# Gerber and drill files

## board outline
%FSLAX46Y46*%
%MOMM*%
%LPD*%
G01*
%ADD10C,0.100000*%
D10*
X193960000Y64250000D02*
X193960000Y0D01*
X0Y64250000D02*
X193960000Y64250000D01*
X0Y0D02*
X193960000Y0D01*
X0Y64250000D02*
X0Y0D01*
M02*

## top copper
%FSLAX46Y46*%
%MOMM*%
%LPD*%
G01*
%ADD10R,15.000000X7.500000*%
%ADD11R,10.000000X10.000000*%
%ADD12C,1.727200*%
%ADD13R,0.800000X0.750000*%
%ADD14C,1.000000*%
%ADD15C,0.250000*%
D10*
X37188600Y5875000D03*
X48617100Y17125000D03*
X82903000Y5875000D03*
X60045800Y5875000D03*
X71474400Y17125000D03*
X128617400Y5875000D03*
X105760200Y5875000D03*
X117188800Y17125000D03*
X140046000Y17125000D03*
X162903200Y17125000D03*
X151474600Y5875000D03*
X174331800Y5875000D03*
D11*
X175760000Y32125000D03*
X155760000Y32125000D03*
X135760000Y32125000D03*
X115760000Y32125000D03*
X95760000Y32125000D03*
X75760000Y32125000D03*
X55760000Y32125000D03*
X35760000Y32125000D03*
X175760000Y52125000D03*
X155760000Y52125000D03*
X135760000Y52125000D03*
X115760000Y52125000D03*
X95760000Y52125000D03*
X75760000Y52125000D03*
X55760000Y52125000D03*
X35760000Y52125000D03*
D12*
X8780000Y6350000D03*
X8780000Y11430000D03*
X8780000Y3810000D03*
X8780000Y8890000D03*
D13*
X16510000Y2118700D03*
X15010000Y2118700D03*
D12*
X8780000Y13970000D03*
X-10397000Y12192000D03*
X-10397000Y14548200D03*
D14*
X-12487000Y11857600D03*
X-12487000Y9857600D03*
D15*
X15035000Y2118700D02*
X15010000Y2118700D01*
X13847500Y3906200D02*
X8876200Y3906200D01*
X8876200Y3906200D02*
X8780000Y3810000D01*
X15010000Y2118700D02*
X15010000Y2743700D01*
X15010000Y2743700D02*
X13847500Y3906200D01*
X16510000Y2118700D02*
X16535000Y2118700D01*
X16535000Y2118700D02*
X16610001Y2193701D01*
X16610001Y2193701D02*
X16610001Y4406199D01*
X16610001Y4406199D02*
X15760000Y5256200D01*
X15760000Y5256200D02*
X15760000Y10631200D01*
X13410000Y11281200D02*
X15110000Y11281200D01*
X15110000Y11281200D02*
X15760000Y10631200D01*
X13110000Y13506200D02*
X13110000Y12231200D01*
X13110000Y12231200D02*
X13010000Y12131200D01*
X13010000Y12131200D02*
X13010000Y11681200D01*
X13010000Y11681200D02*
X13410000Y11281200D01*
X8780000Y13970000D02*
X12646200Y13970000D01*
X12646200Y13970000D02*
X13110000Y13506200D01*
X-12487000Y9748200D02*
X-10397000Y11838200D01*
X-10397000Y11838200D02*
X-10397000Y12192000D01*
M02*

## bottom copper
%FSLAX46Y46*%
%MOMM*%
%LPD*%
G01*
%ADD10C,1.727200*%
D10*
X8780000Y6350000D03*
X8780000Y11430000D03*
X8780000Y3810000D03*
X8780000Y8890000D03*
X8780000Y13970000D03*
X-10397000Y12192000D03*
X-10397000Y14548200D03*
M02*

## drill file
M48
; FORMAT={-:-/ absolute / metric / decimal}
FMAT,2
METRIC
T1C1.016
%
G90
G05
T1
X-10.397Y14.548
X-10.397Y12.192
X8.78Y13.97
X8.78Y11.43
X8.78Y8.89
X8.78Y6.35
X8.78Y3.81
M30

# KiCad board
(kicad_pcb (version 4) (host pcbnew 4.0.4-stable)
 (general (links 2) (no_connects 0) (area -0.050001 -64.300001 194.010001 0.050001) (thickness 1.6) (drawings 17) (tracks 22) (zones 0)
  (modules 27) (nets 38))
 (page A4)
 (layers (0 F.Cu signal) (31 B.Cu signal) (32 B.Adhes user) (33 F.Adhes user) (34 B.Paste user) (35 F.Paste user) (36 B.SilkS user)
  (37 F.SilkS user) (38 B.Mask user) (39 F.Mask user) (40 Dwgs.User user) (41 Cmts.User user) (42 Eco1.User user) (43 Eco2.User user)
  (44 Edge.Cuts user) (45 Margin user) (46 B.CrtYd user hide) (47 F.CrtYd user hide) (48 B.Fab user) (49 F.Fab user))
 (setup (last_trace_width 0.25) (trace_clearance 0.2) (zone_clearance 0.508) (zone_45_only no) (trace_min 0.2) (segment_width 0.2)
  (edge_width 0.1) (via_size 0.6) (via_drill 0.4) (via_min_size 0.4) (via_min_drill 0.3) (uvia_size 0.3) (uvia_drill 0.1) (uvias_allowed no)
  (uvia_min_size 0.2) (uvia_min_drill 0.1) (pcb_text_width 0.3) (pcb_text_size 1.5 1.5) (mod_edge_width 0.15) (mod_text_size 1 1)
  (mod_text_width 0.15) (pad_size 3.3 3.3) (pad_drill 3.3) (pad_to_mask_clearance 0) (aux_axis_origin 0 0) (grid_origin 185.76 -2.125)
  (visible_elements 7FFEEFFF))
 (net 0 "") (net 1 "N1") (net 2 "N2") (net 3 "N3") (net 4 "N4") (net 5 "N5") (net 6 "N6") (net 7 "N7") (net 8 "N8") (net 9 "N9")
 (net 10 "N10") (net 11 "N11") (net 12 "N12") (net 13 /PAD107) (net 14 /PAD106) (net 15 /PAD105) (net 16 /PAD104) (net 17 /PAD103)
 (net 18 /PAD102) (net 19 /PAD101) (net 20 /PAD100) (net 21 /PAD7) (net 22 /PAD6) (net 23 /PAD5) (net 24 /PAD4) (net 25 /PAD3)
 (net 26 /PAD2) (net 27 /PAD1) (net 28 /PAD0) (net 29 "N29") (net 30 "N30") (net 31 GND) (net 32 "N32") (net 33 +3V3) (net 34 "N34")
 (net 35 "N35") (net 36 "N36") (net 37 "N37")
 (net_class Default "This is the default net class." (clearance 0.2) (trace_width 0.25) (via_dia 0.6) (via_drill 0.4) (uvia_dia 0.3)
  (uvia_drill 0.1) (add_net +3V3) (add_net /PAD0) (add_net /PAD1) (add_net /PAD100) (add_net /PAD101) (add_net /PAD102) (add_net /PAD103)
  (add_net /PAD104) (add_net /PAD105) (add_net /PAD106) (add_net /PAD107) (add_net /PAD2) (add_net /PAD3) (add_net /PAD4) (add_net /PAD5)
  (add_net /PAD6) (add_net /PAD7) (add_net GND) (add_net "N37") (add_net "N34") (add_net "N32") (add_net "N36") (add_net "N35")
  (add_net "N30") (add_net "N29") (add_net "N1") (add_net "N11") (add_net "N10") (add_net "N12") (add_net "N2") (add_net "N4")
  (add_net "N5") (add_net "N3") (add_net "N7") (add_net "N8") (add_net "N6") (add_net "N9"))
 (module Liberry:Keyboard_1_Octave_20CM (layer F.Cu) (at 25.76 -2.125)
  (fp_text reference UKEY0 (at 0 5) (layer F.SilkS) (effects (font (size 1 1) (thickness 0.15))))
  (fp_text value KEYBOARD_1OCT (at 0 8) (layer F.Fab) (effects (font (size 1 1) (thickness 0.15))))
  (pad 1 smd rect (at 11.4286 -3.75) (size 15 7.5) (layers F.Cu F.Paste F.Mask) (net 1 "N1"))
  (pad 2 smd rect (at 22.8571 -15) (size 15 7.5) (layers F.Cu F.Paste F.Mask) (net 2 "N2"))
  (pad 5 smd rect (at 57.143 -3.75) (size 15 7.5) (layers F.Cu F.Paste F.Mask) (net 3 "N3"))
  (pad 3 smd rect (at 34.2858 -3.75) (size 15 7.5) (layers F.Cu F.Paste F.Mask) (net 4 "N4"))
  (pad 4 smd rect (at 45.7144 -15) (size 15 7.5) (layers F.Cu F.Paste F.Mask) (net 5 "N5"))
  (pad 8 smd rect (at 102.8574 -3.75) (size 15 7.5) (layers F.Cu F.Paste F.Mask) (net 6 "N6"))
  (pad 6 smd rect (at 80.0002 -3.75) (size 15 7.5) (layers F.Cu F.Paste F.Mask) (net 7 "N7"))
  (pad 7 smd rect (at 91.4288 -15) (size 15 7.5) (layers F.Cu F.Paste F.Mask) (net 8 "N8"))
  (pad 9 smd rect (at 114.286 -15) (size 15 7.5) (layers F.Cu F.Paste F.Mask) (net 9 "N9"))
  (pad 11 smd rect (at 137.1432 -15) (size 15 7.5) (layers F.Cu F.Paste F.Mask) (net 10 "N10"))
  (pad 10 smd rect (at 125.7146 -3.75) (size 15 7.5) (layers F.Cu F.Paste F.Mask) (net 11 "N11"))
  (pad 12 smd rect (at 148.5718 -3.75) (size 15 7.5) (layers F.Cu F.Paste F.Mask) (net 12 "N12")))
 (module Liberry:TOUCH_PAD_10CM (layer F.Cu) (at 175.76 -32.125)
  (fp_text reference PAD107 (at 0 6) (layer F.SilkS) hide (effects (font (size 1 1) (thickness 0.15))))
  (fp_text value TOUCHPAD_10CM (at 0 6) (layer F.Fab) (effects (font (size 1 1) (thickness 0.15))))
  (pad 1 smd rect (at 0 0) (size 10 10) (layers F.Cu) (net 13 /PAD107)))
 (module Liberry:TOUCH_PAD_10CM (layer F.Cu) (at 155.76 -32.125)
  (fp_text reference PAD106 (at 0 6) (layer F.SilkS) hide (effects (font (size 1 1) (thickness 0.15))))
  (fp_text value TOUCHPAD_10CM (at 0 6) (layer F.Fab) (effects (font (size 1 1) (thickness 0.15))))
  (pad 1 smd rect (at 0 0) (size 10 10) (layers F.Cu) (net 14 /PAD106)))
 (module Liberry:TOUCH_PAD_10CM (layer F.Cu) (at 135.76 -32.125)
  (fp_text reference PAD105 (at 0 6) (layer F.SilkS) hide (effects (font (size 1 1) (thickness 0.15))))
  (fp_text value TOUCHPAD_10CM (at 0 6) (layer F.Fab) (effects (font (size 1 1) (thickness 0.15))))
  (pad 1 smd rect (at 0 0) (size 10 10) (layers F.Cu) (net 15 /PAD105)))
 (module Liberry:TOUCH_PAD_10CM (layer F.Cu) (at 115.76 -32.125)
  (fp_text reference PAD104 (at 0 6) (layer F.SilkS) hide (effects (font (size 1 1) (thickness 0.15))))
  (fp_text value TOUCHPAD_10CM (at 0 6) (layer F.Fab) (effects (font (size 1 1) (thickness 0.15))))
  (pad 1 smd rect (at 0 0) (size 10 10) (layers F.Cu) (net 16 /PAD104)))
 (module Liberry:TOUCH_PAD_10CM (layer F.Cu) (at 95.76 -32.125)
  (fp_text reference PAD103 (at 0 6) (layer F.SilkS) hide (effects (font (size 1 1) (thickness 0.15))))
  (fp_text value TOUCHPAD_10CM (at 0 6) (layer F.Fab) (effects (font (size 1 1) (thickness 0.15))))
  (pad 1 smd rect (at 0 0) (size 10 10) (layers F.Cu) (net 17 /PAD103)))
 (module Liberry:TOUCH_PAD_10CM (layer F.Cu) (at 75.76 -32.125)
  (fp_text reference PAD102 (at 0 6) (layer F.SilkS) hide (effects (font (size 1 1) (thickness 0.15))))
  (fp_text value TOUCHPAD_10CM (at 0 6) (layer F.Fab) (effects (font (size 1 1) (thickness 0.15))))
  (pad 1 smd rect (at 0 0) (size 10 10) (layers F.Cu) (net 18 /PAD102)))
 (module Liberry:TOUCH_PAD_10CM (layer F.Cu) (at 55.76 -32.125)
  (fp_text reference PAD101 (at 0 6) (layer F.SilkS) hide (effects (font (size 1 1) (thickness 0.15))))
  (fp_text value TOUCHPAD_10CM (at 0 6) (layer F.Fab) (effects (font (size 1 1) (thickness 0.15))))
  (pad 1 smd rect (at 0 0) (size 10 10) (layers F.Cu) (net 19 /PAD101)))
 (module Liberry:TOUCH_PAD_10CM (layer F.Cu) (at 35.76 -32.125)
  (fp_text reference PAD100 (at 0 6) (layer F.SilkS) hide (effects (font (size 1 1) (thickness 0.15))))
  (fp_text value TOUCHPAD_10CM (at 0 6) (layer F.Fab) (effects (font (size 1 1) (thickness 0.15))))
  (pad 1 smd rect (at 0 0) (size 10 10) (layers F.Cu) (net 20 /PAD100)))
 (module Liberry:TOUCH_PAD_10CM (layer F.Cu) (at 175.76 -52.125)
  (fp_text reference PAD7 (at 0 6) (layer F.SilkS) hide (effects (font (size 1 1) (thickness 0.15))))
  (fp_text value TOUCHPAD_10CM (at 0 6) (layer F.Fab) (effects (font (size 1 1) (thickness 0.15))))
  (pad 1 smd rect (at 0 0) (size 10 10) (layers F.Cu) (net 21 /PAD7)))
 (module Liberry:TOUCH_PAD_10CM (layer F.Cu) (at 155.76 -52.125)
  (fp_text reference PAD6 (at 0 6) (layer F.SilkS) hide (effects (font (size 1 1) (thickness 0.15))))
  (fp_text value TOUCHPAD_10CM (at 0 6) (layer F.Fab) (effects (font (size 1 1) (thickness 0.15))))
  (pad 1 smd rect (at 0 0) (size 10 10) (layers F.Cu) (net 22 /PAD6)))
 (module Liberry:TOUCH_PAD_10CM (layer F.Cu) (at 135.76 -52.125)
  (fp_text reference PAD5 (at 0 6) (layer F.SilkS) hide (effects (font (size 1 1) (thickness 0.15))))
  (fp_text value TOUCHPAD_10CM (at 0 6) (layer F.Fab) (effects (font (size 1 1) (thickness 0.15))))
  (pad 1 smd rect (at 0 0) (size 10 10) (layers F.Cu) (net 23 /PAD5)))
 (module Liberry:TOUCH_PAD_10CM (layer F.Cu) (at 115.76 -52.125)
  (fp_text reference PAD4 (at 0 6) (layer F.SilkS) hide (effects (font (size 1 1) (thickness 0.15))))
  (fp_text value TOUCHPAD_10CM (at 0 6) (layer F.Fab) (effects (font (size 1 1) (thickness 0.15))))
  (pad 1 smd rect (at 0 0) (size 10 10) (layers F.Cu) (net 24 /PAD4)))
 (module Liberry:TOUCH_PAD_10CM (layer F.Cu) (at 95.76 -52.125)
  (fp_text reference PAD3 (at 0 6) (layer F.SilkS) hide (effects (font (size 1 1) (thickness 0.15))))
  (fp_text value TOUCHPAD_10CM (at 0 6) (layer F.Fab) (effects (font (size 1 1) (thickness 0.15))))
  (pad 1 smd rect (at 0 0) (size 10 10) (layers F.Cu) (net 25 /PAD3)))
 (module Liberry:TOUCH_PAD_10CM (layer F.Cu) (at 75.76 -52.125)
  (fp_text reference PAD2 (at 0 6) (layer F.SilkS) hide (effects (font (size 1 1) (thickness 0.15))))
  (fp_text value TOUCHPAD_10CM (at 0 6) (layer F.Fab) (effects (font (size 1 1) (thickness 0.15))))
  (pad 1 smd rect (at 0 0) (size 10 10) (layers F.Cu) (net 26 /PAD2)))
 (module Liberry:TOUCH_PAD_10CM (layer F.Cu) (at 55.76 -52.125)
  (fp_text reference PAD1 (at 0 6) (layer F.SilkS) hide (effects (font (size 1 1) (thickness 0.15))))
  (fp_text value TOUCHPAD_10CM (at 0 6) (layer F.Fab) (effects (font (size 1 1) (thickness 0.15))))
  (pad 1 smd rect (at 0 0) (size 10 10) (layers F.Cu) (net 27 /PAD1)))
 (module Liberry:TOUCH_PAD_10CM (layer F.Cu) (at 35.76 -52.125)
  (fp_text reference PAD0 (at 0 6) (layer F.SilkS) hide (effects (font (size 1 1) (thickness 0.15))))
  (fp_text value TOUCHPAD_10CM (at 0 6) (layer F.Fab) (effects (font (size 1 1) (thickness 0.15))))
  (pad 1 smd rect (at 0 0) (size 10 10) (layers F.Cu) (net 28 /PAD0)))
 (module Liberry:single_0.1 (layer F.Cu) (at 8.78 -6.35)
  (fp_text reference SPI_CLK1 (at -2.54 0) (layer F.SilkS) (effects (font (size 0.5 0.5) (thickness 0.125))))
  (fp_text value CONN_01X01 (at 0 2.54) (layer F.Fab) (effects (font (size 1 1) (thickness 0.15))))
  (pad 1 thru_hole circle (at 0 0) (size 1.7272 1.7272) (drill 1.016) (layers *.Cu *.Mask) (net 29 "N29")))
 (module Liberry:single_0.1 (layer F.Cu) (at 8.78 -11.43)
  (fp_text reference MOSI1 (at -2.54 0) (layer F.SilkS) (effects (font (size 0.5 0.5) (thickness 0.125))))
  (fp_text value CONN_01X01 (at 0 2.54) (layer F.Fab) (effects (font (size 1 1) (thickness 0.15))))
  (pad 1 thru_hole circle (at 0 0) (size 1.7272 1.7272) (drill 1.016) (layers *.Cu *.Mask) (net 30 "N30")))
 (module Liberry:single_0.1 (layer F.Cu) (at 8.78 -3.81)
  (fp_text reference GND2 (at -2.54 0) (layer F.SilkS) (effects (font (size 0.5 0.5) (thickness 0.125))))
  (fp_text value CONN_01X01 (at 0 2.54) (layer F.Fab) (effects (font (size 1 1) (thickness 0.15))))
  (pad 1 thru_hole circle (at 0 0) (size 1.7272 1.7272) (drill 1.016) (layers *.Cu *.Mask) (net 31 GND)))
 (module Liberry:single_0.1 (layer F.Cu) (at 8.78 -8.89)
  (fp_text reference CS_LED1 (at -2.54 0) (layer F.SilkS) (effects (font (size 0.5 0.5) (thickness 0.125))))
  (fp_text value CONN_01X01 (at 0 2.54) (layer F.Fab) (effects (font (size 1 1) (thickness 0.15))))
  (pad 1 thru_hole circle (at 0 0) (size 1.7272 1.7272) (drill 1.016) (layers *.Cu *.Mask) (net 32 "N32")))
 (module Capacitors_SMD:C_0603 (layer F.Cu) (at 15.76 -2.1187 180)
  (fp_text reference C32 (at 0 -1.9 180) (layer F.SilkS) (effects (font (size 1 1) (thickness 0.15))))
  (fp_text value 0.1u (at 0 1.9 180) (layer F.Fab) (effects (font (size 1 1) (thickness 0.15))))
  (pad 1 smd rect (at -0.75 0 180) (size 0.8 0.75) (layers F.Cu F.Paste F.Mask) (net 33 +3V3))
  (pad 2 smd rect (at 0.75 0 180) (size 0.8 0.75) (layers F.Cu F.Paste F.Mask) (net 31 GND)))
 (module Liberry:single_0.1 (layer F.Cu) (at 8.78 -13.97)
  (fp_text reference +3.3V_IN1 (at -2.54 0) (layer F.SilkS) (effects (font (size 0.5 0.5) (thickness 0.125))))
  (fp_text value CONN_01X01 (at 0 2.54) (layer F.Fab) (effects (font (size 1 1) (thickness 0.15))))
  (pad 1 thru_hole circle (at 0 0) (size 1.7272 1.7272) (drill 1.016) (layers *.Cu *.Mask) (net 33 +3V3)))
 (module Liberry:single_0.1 (layer F.Cu) (at -10.397 -12.192)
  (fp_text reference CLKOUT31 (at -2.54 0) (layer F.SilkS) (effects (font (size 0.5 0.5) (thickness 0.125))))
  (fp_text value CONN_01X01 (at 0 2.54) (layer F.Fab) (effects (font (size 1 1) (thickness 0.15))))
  (pad 1 thru_hole circle (at 0 0) (size 1.7272 1.7272) (drill 1.016) (layers *.Cu *.Mask) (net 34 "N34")))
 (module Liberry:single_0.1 (layer F.Cu) (at -10.397 -14.5482)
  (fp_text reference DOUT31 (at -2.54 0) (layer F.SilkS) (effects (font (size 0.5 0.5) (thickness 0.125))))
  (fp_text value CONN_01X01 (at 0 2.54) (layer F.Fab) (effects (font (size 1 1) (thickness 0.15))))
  (pad 1 thru_hole circle (at 0 0) (size 1.7272 1.7272) (drill 1.016) (layers *.Cu *.Mask) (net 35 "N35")))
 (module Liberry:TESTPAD (layer F.Cu) (at -12.487 -11.8576)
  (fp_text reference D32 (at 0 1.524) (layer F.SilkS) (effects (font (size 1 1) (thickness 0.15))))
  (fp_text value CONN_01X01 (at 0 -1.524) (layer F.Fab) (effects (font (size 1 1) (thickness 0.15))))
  (pad 1 smd circle (at 0 0 270) (size 1 1) (layers F.Cu F.Paste F.Mask) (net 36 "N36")))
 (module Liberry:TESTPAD (layer F.Cu) (at -12.487 -9.8576)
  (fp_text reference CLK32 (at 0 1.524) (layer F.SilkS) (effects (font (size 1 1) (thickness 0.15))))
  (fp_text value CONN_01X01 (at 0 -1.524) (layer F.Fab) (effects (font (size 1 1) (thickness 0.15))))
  (pad 1 smd circle (at 0 0 270) (size 1 1) (layers F.Cu F.Paste F.Mask) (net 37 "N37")))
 (gr_line (start 193.96 -64.25) (end 193.96 0) (layer Edge.Cuts) (width 0.1))
 (gr_line (start 0 -64.25) (end 193.96 -64.25) (layer Edge.Cuts) (width 0.1))
 (gr_line (start 0 0) (end 193.96 0) (layer Edge.Cuts) (width 0.1))
 (gr_line (start 0 -64.25) (end 0 0) (layer Edge.Cuts) (width 0.1))
 (segment (start 25.76 -2.125) (end 25.76 -32.125) (width 0.25) (layer Dwgs.User) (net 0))
 (segment (start 185.76 -2.125) (end 25.76 -2.125) (width 0.25) (layer Dwgs.User) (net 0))
 (segment (start 15.035 -2.1187) (end 15.01 -2.1187) (width 0.25) (layer F.Cu) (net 31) (status 30))
 (segment (start 13.8475 -3.9062) (end 8.8762 -3.9062) (width 0.25) (layer F.Cu) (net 31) (status 20))
 (segment (start 8.8762 -3.9062) (end 8.78 -3.81) (width 0.25) (layer F.Cu) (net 31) (status 30))
 (segment (start 15.01 -2.1187) (end 15.01 -2.7437) (width 0.25) (layer F.Cu) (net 31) (status 10))
 (segment (start 15.01 -2.7437) (end 13.8475 -3.9062) (width 0.25) (layer F.Cu) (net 31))
 (segment (start 16.51 -2.1187) (end 16.535 -2.1187) (width 0.25) (layer F.Cu) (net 33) (status 30))
 (segment (start 16.535 -2.1187) (end 16.610001 -2.193701) (width 0.25) (layer F.Cu) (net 33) (status 30))
 (segment (start 16.610001 -2.193701) (end 16.610001 -4.406199) (width 0.25) (layer F.Cu) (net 33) (status 10))
 (segment (start 16.610001 -4.406199) (end 15.76 -5.2562) (width 0.25) (layer F.Cu) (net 33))
 (segment (start 15.76 -5.2562) (end 15.76 -10.6312) (width 0.25) (layer F.Cu) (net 33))
 (segment (start 13.41 -11.2812) (end 15.11 -11.2812) (width 0.25) (layer F.Cu) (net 33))
 (segment (start 15.11 -11.2812) (end 15.76 -10.6312) (width 0.25) (layer F.Cu) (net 33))
 (segment (start 13.11 -13.5062) (end 13.11 -12.2312) (width 0.25) (layer F.Cu) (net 33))
 (segment (start 13.11 -12.2312) (end 13.01 -12.1312) (width 0.25) (layer F.Cu) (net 33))
 (segment (start 13.01 -12.1312) (end 13.01 -11.6812) (width 0.25) (layer F.Cu) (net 33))
 (segment (start 13.01 -11.6812) (end 13.41 -11.2812) (width 0.25) (layer F.Cu) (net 33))
 (segment (start 8.78 -13.97) (end 12.6462 -13.97) (width 0.25) (layer F.Cu) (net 33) (status 10))
 (segment (start 12.6462 -13.97) (end 13.11 -13.5062) (width 0.25) (layer F.Cu) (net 33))
 (segment (start -12.487 -9.7482) (end -10.397 -11.8382) (width 0.25) (layer F.Cu) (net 37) (status 30))
 (segment (start -10.397 -11.8382) (end -10.397 -12.192) (width 0.25) (layer F.Cu) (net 34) (status 30)))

